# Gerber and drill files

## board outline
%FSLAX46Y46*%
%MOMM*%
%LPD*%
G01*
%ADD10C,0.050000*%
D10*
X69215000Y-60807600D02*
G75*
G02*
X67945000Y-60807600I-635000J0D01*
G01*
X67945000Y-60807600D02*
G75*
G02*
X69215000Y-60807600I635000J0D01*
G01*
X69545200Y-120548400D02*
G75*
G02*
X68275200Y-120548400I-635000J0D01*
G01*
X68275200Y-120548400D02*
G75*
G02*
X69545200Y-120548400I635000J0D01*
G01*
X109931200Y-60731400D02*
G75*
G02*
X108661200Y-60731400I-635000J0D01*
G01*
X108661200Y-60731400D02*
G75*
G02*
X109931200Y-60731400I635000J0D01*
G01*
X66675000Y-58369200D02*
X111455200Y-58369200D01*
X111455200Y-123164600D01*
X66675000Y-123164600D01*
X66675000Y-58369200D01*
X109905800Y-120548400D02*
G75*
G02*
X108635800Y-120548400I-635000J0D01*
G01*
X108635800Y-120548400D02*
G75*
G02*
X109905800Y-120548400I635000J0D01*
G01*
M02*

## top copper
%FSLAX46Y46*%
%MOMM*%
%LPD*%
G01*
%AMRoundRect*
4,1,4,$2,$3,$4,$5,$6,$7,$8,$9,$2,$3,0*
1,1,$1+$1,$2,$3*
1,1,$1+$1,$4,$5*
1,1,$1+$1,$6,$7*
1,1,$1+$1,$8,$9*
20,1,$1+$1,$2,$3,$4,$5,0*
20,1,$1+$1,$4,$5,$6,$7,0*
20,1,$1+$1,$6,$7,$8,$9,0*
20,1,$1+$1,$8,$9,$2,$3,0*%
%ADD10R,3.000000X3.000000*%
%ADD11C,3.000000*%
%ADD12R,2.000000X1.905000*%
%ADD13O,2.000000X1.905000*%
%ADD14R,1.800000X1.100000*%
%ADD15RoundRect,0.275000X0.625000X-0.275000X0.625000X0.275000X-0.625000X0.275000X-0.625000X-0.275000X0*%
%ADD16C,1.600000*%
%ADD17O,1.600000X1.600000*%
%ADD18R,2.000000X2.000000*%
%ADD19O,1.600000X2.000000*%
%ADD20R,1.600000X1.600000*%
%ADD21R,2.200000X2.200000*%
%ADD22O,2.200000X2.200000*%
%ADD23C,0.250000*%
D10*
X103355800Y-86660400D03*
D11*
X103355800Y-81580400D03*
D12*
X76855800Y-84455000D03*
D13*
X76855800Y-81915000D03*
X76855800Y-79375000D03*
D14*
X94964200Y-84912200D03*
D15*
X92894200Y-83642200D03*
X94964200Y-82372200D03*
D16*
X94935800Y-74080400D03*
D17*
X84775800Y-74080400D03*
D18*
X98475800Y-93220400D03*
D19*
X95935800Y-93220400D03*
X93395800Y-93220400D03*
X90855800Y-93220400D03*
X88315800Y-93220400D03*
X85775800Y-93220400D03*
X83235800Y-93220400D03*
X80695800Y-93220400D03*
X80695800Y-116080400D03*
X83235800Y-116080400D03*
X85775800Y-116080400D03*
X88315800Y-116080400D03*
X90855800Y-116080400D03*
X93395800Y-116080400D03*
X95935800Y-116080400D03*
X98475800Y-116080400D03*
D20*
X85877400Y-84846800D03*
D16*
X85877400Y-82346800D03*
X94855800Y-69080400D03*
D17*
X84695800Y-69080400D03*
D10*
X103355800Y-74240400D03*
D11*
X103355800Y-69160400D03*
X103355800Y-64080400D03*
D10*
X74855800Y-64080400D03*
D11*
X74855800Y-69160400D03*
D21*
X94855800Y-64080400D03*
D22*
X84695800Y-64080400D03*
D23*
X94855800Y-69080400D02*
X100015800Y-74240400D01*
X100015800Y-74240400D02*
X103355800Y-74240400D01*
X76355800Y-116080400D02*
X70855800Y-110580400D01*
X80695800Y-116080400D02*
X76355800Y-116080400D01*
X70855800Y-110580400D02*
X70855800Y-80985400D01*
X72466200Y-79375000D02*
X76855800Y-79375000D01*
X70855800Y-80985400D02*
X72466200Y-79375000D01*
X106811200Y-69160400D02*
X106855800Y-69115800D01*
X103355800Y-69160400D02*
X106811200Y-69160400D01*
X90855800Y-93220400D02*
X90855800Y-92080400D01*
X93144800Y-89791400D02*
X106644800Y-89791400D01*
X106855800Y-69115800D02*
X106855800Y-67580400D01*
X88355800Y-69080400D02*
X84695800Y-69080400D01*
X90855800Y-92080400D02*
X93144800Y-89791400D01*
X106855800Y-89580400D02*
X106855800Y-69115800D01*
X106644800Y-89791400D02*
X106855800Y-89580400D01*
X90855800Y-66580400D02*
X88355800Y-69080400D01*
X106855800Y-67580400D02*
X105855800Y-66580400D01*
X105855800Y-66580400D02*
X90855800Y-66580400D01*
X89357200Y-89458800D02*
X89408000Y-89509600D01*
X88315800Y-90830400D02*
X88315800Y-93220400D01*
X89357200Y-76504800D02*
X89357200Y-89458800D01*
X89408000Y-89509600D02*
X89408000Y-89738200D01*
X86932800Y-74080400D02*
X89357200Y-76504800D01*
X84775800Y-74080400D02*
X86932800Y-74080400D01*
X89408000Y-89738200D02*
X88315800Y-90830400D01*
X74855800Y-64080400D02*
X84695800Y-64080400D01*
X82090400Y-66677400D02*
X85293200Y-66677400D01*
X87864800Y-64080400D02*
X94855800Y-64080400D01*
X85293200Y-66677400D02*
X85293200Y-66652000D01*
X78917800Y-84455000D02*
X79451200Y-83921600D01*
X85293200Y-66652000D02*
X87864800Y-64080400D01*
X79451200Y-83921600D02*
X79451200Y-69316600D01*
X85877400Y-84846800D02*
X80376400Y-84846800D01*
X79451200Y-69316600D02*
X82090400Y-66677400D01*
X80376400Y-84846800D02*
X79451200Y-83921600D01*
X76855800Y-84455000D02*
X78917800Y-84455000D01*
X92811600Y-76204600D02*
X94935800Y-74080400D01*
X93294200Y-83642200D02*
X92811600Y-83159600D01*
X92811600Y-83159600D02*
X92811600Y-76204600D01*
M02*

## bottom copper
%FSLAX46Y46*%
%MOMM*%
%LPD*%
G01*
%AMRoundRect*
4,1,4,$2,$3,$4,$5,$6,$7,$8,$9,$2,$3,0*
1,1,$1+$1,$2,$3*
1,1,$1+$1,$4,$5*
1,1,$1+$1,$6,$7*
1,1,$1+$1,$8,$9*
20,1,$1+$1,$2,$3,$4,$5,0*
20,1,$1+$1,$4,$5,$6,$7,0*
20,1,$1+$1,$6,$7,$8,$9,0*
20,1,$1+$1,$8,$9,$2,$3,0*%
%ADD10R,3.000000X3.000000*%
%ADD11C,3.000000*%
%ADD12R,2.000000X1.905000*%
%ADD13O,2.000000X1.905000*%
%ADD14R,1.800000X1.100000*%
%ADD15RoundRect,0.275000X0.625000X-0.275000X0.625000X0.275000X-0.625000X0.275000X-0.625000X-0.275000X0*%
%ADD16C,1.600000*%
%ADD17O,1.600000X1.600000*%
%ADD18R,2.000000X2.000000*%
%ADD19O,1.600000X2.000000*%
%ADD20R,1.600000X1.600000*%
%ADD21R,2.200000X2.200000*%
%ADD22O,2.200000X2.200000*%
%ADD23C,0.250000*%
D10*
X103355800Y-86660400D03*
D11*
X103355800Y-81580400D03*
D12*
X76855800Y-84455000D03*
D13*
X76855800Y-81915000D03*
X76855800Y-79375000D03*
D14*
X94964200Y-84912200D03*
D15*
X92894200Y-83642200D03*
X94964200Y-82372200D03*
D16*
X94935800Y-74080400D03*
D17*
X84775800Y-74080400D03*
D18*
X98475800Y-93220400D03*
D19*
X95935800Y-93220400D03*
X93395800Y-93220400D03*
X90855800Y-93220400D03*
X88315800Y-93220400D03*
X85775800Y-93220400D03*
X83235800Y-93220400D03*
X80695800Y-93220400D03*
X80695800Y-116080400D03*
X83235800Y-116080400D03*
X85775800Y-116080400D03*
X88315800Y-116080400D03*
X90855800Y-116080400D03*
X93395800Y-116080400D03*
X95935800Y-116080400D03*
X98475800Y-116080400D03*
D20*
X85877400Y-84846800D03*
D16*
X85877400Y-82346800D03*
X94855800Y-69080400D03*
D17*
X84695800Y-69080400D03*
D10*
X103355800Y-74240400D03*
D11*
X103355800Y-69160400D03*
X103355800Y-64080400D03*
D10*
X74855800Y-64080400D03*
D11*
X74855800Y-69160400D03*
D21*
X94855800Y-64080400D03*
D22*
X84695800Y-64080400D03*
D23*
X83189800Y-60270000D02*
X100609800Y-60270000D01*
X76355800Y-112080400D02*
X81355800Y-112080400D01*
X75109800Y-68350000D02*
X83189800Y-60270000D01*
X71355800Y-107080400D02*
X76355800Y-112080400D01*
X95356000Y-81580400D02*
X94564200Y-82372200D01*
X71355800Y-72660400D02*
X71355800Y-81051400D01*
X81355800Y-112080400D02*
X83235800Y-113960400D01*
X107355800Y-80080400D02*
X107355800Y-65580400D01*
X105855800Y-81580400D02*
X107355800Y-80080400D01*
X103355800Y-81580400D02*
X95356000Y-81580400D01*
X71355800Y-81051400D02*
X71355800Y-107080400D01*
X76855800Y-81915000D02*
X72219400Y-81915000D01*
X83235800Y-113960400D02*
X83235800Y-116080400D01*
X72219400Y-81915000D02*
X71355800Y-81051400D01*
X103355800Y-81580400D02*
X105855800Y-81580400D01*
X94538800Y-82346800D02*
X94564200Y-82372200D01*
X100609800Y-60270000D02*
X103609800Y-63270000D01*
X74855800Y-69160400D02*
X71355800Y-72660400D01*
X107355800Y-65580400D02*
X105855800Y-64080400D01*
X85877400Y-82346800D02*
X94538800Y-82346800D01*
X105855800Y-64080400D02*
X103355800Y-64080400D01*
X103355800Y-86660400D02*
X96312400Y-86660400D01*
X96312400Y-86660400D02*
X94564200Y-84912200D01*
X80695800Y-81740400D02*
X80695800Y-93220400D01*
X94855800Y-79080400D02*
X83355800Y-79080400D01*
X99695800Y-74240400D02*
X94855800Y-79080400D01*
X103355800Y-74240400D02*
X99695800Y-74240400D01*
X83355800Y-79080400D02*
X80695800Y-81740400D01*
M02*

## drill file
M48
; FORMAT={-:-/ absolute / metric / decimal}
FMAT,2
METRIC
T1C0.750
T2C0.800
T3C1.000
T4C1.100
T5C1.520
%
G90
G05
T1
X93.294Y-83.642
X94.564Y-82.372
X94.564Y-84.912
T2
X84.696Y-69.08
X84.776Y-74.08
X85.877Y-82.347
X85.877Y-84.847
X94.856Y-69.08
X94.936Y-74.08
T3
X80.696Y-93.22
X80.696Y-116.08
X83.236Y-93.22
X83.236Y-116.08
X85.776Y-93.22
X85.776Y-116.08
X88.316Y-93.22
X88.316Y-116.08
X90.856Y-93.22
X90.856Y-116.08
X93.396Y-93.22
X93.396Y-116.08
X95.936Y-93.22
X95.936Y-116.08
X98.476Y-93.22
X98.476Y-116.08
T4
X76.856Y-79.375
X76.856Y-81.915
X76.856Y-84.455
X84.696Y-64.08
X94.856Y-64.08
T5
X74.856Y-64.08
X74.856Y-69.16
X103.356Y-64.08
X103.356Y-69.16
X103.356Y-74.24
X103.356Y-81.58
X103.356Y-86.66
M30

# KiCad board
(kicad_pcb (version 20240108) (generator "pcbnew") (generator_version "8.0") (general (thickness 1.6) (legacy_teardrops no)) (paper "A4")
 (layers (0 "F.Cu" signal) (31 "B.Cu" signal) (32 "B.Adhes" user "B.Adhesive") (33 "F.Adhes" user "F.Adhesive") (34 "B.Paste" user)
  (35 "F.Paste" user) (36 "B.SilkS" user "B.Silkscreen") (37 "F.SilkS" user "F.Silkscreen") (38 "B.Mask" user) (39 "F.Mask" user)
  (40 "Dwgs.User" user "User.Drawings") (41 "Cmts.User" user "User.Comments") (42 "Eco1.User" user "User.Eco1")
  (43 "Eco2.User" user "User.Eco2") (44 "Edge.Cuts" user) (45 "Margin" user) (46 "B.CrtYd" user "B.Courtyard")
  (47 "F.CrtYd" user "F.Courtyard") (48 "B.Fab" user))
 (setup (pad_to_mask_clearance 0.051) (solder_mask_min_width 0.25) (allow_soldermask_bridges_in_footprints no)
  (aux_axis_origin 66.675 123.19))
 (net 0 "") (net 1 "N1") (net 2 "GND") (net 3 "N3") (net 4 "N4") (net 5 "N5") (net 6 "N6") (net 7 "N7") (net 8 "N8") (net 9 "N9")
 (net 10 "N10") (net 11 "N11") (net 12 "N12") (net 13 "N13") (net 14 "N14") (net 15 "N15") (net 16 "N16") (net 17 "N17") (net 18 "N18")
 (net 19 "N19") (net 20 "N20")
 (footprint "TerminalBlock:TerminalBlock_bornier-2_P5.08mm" (layer "F.Cu") (at 103.3558 86.6604 90)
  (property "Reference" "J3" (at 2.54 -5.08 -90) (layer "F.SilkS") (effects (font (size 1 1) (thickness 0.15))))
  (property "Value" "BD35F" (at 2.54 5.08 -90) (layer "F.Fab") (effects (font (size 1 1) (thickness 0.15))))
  (pad "1" thru_hole rect (at 0 0 90) (size 3 3) (drill 1.52) (layers "*.Cu" "*.Mask") (remove_unused_layers no) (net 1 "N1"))
  (pad "2" thru_hole circle (at 5.08 0 90) (size 3 3) (drill 1.52) (layers "*.Cu" "*.Mask") (remove_unused_layers no) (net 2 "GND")))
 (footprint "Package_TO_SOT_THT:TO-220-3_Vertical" (layer "F.Cu") (at 76.8558 84.455 90)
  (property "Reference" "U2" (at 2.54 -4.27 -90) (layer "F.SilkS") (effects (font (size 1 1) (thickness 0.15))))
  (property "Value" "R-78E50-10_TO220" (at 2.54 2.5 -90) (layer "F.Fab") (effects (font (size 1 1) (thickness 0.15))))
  (pad "1" thru_hole rect (at 0 0 90) (size 1.905 2) (drill 1.1) (layers "*.Cu" "*.Mask") (remove_unused_layers no) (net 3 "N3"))
  (pad "2" thru_hole oval (at 2.54 0 90) (size 1.905 2) (drill 1.1) (layers "*.Cu" "*.Mask") (remove_unused_layers no) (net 2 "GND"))
  (pad "3" thru_hole oval (at 5.08 0 90) (size 1.905 2) (drill 1.1) (layers "*.Cu" "*.Mask") (remove_unused_layers no) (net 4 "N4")))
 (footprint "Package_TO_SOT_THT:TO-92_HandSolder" (layer "F.Cu") (at 94.5642 84.9122 90)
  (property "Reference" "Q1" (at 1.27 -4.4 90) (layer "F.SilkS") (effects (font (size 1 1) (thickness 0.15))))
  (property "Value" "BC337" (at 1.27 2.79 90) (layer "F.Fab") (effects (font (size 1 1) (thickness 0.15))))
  (pad "1" thru_hole rect (at 0 0 90) (size 1.1 1.8) (drill 0.75 (offset 0 0.4)) (layers "*.Cu" "*.Mask") (remove_unused_layers no)
   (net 1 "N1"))
  (pad "2" thru_hole roundrect (at 1.27 -1.27 90) (size 1.1 1.8) (drill 0.75 (offset 0 -0.4)) (layers "*.Cu" "*.Mask")
   (remove_unused_layers no) (roundrect_rratio 0.25) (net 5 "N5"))
  (pad "3" thru_hole roundrect (at 2.54 0 90) (size 1.1 1.8) (drill 0.75 (offset 0 0.4)) (layers "*.Cu" "*.Mask") (remove_unused_layers no)
   (roundrect_rratio 0.25) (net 2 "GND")))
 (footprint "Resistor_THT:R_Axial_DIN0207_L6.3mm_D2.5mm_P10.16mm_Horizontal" (layer "F.Cu") (at 94.9358 74.0804 180)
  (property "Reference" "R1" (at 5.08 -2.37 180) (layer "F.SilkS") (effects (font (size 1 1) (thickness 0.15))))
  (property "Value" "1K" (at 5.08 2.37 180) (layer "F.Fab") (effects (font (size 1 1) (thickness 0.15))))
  (pad "1" thru_hole circle (at 0 0 180) (size 1.6 1.6) (drill 0.8) (layers "*.Cu" "*.Mask") (remove_unused_layers no) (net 5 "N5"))
  (pad "2" thru_hole oval (at 10.16 0 180) (size 1.6 1.6) (drill 0.8) (layers "*.Cu" "*.Mask") (remove_unused_layers no) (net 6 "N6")))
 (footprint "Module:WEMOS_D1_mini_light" (layer "F.Cu") (at 98.4758 93.2204 -90)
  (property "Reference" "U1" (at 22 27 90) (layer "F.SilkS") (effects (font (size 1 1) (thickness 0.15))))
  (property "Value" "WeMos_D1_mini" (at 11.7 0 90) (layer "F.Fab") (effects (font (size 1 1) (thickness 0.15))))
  (pad "1" thru_hole rect (at 0 0 270) (size 2 2) (drill 1) (layers "*.Cu" "*.Mask") (remove_unused_layers no) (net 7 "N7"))
  (pad "2" thru_hole oval (at 0 2.54 270) (size 2 1.6) (drill 1) (layers "*.Cu" "*.Mask") (remove_unused_layers no) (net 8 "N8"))
  (pad "3" thru_hole oval (at 0 5.08 270) (size 2 1.6) (drill 1) (layers "*.Cu" "*.Mask") (remove_unused_layers no) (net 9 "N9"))
  (pad "4" thru_hole oval (at 0 7.62 270) (size 2 1.6) (drill 1) (layers "*.Cu" "*.Mask") (remove_unused_layers no) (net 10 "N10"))
  (pad "5" thru_hole oval (at 0 10.16 270) (size 2 1.6) (drill 1) (layers "*.Cu" "*.Mask") (remove_unused_layers no) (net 6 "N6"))
  (pad "6" thru_hole oval (at 0 12.7 270) (size 2 1.6) (drill 1) (layers "*.Cu" "*.Mask") (remove_unused_layers no) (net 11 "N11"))
  (pad "7" thru_hole oval (at 0 15.24 270) (size 2 1.6) (drill 1) (layers "*.Cu" "*.Mask") (remove_unused_layers no) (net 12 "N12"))
  (pad "8" thru_hole oval (at 0 17.78 270) (size 2 1.6) (drill 1) (layers "*.Cu" "*.Mask") (remove_unused_layers no) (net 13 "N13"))
  (pad "9" thru_hole oval (at 22.86 17.78 270) (size 2 1.6) (drill 1) (layers "*.Cu" "*.Mask") (remove_unused_layers no) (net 4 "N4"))
  (pad "10" thru_hole oval (at 22.86 15.24 270) (size 2 1.6) (drill 1) (layers "*.Cu" "*.Mask") (remove_unused_layers no) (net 2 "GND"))
  (pad "11" thru_hole oval (at 22.86 12.7 270) (size 2 1.6) (drill 1) (layers "*.Cu" "*.Mask") (remove_unused_layers no) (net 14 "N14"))
  (pad "12" thru_hole oval (at 22.86 10.16 270) (size 2 1.6) (drill 1) (layers "*.Cu" "*.Mask") (remove_unused_layers no) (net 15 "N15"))
  (pad "13" thru_hole oval (at 22.86 7.62 270) (size 2 1.6) (drill 1) (layers "*.Cu" "*.Mask") (remove_unused_layers no) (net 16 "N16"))
  (pad "14" thru_hole oval (at 22.86 5.08 270) (size 2 1.6) (drill 1) (layers "*.Cu" "*.Mask") (remove_unused_layers no) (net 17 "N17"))
  (pad "15" thru_hole oval (at 22.86 2.54 270) (size 2 1.6) (drill 1) (layers "*.Cu" "*.Mask") (remove_unused_layers no) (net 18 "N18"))
  (pad "16" thru_hole oval (at 22.86 0 270) (size 2 1.6) (drill 1) (layers "*.Cu" "*.Mask") (remove_unused_layers no) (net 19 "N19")))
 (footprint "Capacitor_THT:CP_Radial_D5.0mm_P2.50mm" (layer "F.Cu") (at 85.8774 84.8468 90)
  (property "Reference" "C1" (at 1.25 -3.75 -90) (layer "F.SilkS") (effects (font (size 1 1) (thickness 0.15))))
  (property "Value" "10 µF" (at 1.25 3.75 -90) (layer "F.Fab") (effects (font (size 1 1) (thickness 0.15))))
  (pad "1" thru_hole rect (at 0 0 90) (size 1.6 1.6) (drill 0.8) (layers "*.Cu" "*.Mask") (remove_unused_layers no) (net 3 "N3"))
  (pad "2" thru_hole circle (at 2.5 0 90) (size 1.6 1.6) (drill 0.8) (layers "*.Cu" "*.Mask") (remove_unused_layers no) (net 2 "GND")))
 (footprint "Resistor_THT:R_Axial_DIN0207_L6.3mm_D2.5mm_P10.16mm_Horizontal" (layer "F.Cu") (at 94.8558 69.0804 180)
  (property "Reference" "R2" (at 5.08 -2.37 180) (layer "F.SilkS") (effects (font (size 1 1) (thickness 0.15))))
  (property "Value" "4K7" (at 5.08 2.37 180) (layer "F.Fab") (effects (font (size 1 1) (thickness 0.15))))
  (pad "1" thru_hole circle (at 0 0 180) (size 1.6 1.6) (drill 0.8) (layers "*.Cu" "*.Mask") (remove_unused_layers no) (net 13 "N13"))
  (pad "2" thru_hole oval (at 10.16 0 180) (size 1.6 1.6) (drill 0.8) (layers "*.Cu" "*.Mask") (remove_unused_layers no) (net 10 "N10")))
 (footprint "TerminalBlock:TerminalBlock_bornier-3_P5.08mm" (layer "F.Cu") (at 103.3558 74.2404 90)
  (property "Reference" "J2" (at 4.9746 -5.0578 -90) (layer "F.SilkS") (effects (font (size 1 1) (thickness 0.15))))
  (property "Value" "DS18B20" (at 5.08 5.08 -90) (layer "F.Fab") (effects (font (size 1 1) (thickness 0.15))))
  (pad "1" thru_hole rect (at 0 0 90) (size 3 3) (drill 1.52) (layers "*.Cu" "*.Mask") (remove_unused_layers no) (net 13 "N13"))
  (pad "2" thru_hole circle (at 5.08 0 90) (size 3 3) (drill 1.52) (layers "*.Cu" "*.Mask") (remove_unused_layers no) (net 10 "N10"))
  (pad "3" thru_hole circle (at 10.16 0 90) (size 3 3) (drill 1.52) (layers "*.Cu" "*.Mask") (remove_unused_layers no) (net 2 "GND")))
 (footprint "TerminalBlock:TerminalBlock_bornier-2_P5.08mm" (layer "F.Cu") (at 74.8558 64.0804 -90)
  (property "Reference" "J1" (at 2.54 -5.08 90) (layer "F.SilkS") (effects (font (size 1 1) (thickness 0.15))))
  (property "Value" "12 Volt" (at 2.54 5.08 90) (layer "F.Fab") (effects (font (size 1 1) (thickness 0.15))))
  (pad "1" thru_hole rect (at 0 0 270) (size 3 3) (drill 1.52) (layers "*.Cu" "*.Mask") (remove_unused_layers no) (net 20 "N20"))
  (pad "2" thru_hole circle (at 5.08 0 270) (size 3 3) (drill 1.52) (layers "*.Cu" "*.Mask") (remove_unused_layers no) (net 2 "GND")))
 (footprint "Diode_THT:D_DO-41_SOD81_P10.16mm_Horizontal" (layer "F.Cu") (at 94.8558 64.0804 180)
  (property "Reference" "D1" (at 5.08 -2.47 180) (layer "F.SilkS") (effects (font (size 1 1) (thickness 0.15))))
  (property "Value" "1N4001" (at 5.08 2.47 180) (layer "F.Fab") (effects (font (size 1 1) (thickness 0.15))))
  (pad "1" thru_hole rect (at 0 0 180) (size 2.2 2.2) (drill 1.1) (layers "*.Cu" "*.Mask") (remove_unused_layers no) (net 3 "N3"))
  (pad "2" thru_hole oval (at 10.16 0 180) (size 2.2 2.2) (drill 1.1) (layers "*.Cu" "*.Mask") (remove_unused_layers no) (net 20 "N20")))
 (gr_circle (center 68.58 60.8076) (end 69.215 60.8076) (stroke (width 0.05) (type solid)) (fill none) (layer "Edge.Cuts"))
 (gr_circle (center 68.9102 120.5484) (end 68.9102 119.9134) (stroke (width 0.05) (type solid)) (fill none) (layer "Edge.Cuts"))
 (gr_circle (center 109.2962 60.7314) (end 109.9312 60.7314) (stroke (width 0.05) (type solid)) (fill none) (layer "Edge.Cuts"))
 (gr_rect (start 66.675 58.3692) (end 111.4552 123.1646) (stroke (width 0.05) (type default)) (fill none) (layer "Edge.Cuts"))
 (gr_circle (center 109.2708 120.5484) (end 109.9058 120.5484) (stroke (width 0.05) (type solid)) (fill none) (layer "Edge.Cuts"))
 (segment (start 83.1898 60.27) (end 100.6098 60.27) (width 0.25) (layer "B.Cu") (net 2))
 (segment (start 76.3558 112.0804) (end 81.3558 112.0804) (width 0.25) (layer "B.Cu") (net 2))
 (segment (start 75.1098 68.35) (end 83.1898 60.27) (width 0.25) (layer "B.Cu") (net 2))
 (segment (start 71.3558 107.0804) (end 76.3558 112.0804) (width 0.25) (layer "B.Cu") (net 2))
 (segment (start 95.356 81.5804) (end 94.5642 82.3722) (width 0.25) (layer "B.Cu") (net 2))
 (segment (start 71.3558 72.6604) (end 71.3558 81.0514) (width 0.25) (layer "B.Cu") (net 2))
 (segment (start 81.3558 112.0804) (end 83.2358 113.9604) (width 0.25) (layer "B.Cu") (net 2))
 (segment (start 107.3558 80.0804) (end 107.3558 65.5804) (width 0.25) (layer "B.Cu") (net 2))
 (segment (start 105.8558 81.5804) (end 107.3558 80.0804) (width 0.25) (layer "B.Cu") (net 2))
 (segment (start 103.3558 81.5804) (end 95.356 81.5804) (width 0.25) (layer "B.Cu") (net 2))
 (segment (start 71.3558 81.0514) (end 71.3558 107.0804) (width 0.25) (layer "B.Cu") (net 2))
 (segment (start 76.8558 81.915) (end 72.2194 81.915) (width 0.25) (layer "B.Cu") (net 2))
 (segment (start 83.2358 113.9604) (end 83.2358 116.0804) (width 0.25) (layer "B.Cu") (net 2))
 (segment (start 72.2194 81.915) (end 71.3558 81.0514) (width 0.25) (layer "B.Cu") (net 2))
 (segment (start 103.3558 81.5804) (end 105.8558 81.5804) (width 0.25) (layer "B.Cu") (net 2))
 (segment (start 94.5388 82.3468) (end 94.5642 82.3722) (width 0.25) (layer "B.Cu") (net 2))
 (segment (start 100.6098 60.27) (end 103.6098 63.27) (width 0.25) (layer "B.Cu") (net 2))
 (segment (start 74.8558 69.1604) (end 71.3558 72.6604) (width 0.25) (layer "B.Cu") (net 2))
 (segment (start 107.3558 65.5804) (end 105.8558 64.0804) (width 0.25) (layer "B.Cu") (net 2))
 (segment (start 85.8774 82.3468) (end 94.5388 82.3468) (width 0.25) (layer "B.Cu") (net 2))
 (segment (start 105.8558 64.0804) (end 103.3558 64.0804) (width 0.25) (layer "B.Cu") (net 2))
 (segment (start 103.3558 86.6604) (end 96.3124 86.6604) (width 0.25) (layer "B.Cu") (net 1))
 (segment (start 96.3124 86.6604) (end 94.5642 84.9122) (width 0.25) (layer "B.Cu") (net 1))
 (segment (start 94.8558 69.0804) (end 100.0158 74.2404) (width 0.25) (layer "F.Cu") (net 13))
 (segment (start 100.0158 74.2404) (end 103.3558 74.2404) (width 0.25) (layer "F.Cu") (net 13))
 (segment (start 80.6958 81.7404) (end 80.6958 93.2204) (width 0.25) (layer "B.Cu") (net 13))
 (segment (start 94.8558 79.0804) (end 83.3558 79.0804) (width 0.25) (layer "B.Cu") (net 13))
 (segment (start 99.6958 74.2404) (end 94.8558 79.0804) (width 0.25) (layer "B.Cu") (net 13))
 (segment (start 103.3558 74.2404) (end 99.6958 74.2404) (width 0.25) (layer "B.Cu") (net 13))
 (segment (start 83.3558 79.0804) (end 80.6958 81.7404) (width 0.25) (layer "B.Cu") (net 13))
 (segment (start 76.3558 116.0804) (end 70.8558 110.5804) (width 0.25) (layer "F.Cu") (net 4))
 (segment (start 80.6958 116.0804) (end 76.3558 116.0804) (width 0.25) (layer "F.Cu") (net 4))
 (segment (start 70.8558 110.5804) (end 70.8558 80.9854) (width 0.25) (layer "F.Cu") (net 4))
 (segment (start 72.4662 79.375) (end 76.8558 79.375) (width 0.25) (layer "F.Cu") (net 4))
 (segment (start 70.8558 80.9854) (end 72.4662 79.375) (width 0.25) (layer "F.Cu") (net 4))
 (segment (start 106.8112 69.1604) (end 106.8558 69.1158) (width 0.25) (layer "F.Cu") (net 10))
 (segment (start 103.3558 69.1604) (end 106.8112 69.1604) (width 0.25) (layer "F.Cu") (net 10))
 (segment (start 90.8558 93.2204) (end 90.8558 92.0804) (width 0.25) (layer "F.Cu") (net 10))
 (segment (start 93.1448 89.7914) (end 106.6448 89.7914) (width 0.25) (layer "F.Cu") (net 10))
 (segment (start 106.8558 69.1158) (end 106.8558 67.5804) (width 0.25) (layer "F.Cu") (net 10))
 (segment (start 88.3558 69.0804) (end 84.6958 69.0804) (width 0.25) (layer "F.Cu") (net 10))
 (segment (start 90.8558 92.0804) (end 93.1448 89.7914) (width 0.25) (layer "F.Cu") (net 10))
 (segment (start 106.8558 89.5804) (end 106.8558 69.1158) (width 0.25) (layer "F.Cu") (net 10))
 (segment (start 106.6448 89.7914) (end 106.8558 89.5804) (width 0.25) (layer "F.Cu") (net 10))
 (segment (start 90.8558 66.5804) (end 88.3558 69.0804) (width 0.25) (layer "F.Cu") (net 10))
 (segment (start 106.8558 67.5804) (end 105.8558 66.5804) (width 0.25) (layer "F.Cu") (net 10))
 (segment (start 105.8558 66.5804) (end 90.8558 66.5804) (width 0.25) (layer "F.Cu") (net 10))
 (segment (start 89.3572 89.4588) (end 89.408 89.5096) (width 0.25) (layer "F.Cu") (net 6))
 (segment (start 88.3158 90.8304) (end 88.3158 93.2204) (width 0.25) (layer "F.Cu") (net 6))
 (segment (start 89.3572 76.5048) (end 89.3572 89.4588) (width 0.25) (layer "F.Cu") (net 6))
 (segment (start 89.408 89.5096) (end 89.408 89.7382) (width 0.25) (layer "F.Cu") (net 6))
 (segment (start 86.9328 74.0804) (end 89.3572 76.5048) (width 0.25) (layer "F.Cu") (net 6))
 (segment (start 84.7758 74.0804) (end 86.9328 74.0804) (width 0.25) (layer "F.Cu") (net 6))
 (segment (start 89.408 89.7382) (end 88.3158 90.8304) (width 0.25) (layer "F.Cu") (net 6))
 (segment (start 74.8558 64.0804) (end 84.6958 64.0804) (width 0.25) (layer "F.Cu") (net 20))
 (segment (start 82.0904 66.6774) (end 85.2932 66.6774) (width 0.25) (layer "F.Cu") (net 3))
 (segment (start 87.8648 64.0804) (end 94.8558 64.0804) (width 0.25) (layer "F.Cu") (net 3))
 (segment (start 85.2932 66.6774) (end 85.2932 66.652) (width 0.25) (layer "F.Cu") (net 3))
 (segment (start 78.9178 84.455) (end 79.4512 83.9216) (width 0.25) (layer "F.Cu") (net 3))
 (segment (start 85.2932 66.652) (end 87.8648 64.0804) (width 0.25) (layer "F.Cu") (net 3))
 (segment (start 79.4512 83.9216) (end 79.4512 69.3166) (width 0.25) (layer "F.Cu") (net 3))
 (segment (start 85.8774 84.8468) (end 80.3764 84.8468) (width 0.25) (layer "F.Cu") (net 3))
 (segment (start 79.4512 69.3166) (end 82.0904 66.6774) (width 0.25) (layer "F.Cu") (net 3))
 (segment (start 80.3764 84.8468) (end 79.4512 83.9216) (width 0.25) (layer "F.Cu") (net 3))
 (segment (start 76.8558 84.455) (end 78.9178 84.455) (width 0.25) (layer "F.Cu") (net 3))
 (segment (start 92.8116 76.2046) (end 94.9358 74.0804) (width 0.25) (layer "F.Cu") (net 5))
 (segment (start 93.2942 83.6422) (end 92.8116 83.1596) (width 0.25) (layer "F.Cu") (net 5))
 (segment (start 92.8116 83.1596) (end 92.8116 76.2046) (width 0.25) (layer "F.Cu") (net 5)))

